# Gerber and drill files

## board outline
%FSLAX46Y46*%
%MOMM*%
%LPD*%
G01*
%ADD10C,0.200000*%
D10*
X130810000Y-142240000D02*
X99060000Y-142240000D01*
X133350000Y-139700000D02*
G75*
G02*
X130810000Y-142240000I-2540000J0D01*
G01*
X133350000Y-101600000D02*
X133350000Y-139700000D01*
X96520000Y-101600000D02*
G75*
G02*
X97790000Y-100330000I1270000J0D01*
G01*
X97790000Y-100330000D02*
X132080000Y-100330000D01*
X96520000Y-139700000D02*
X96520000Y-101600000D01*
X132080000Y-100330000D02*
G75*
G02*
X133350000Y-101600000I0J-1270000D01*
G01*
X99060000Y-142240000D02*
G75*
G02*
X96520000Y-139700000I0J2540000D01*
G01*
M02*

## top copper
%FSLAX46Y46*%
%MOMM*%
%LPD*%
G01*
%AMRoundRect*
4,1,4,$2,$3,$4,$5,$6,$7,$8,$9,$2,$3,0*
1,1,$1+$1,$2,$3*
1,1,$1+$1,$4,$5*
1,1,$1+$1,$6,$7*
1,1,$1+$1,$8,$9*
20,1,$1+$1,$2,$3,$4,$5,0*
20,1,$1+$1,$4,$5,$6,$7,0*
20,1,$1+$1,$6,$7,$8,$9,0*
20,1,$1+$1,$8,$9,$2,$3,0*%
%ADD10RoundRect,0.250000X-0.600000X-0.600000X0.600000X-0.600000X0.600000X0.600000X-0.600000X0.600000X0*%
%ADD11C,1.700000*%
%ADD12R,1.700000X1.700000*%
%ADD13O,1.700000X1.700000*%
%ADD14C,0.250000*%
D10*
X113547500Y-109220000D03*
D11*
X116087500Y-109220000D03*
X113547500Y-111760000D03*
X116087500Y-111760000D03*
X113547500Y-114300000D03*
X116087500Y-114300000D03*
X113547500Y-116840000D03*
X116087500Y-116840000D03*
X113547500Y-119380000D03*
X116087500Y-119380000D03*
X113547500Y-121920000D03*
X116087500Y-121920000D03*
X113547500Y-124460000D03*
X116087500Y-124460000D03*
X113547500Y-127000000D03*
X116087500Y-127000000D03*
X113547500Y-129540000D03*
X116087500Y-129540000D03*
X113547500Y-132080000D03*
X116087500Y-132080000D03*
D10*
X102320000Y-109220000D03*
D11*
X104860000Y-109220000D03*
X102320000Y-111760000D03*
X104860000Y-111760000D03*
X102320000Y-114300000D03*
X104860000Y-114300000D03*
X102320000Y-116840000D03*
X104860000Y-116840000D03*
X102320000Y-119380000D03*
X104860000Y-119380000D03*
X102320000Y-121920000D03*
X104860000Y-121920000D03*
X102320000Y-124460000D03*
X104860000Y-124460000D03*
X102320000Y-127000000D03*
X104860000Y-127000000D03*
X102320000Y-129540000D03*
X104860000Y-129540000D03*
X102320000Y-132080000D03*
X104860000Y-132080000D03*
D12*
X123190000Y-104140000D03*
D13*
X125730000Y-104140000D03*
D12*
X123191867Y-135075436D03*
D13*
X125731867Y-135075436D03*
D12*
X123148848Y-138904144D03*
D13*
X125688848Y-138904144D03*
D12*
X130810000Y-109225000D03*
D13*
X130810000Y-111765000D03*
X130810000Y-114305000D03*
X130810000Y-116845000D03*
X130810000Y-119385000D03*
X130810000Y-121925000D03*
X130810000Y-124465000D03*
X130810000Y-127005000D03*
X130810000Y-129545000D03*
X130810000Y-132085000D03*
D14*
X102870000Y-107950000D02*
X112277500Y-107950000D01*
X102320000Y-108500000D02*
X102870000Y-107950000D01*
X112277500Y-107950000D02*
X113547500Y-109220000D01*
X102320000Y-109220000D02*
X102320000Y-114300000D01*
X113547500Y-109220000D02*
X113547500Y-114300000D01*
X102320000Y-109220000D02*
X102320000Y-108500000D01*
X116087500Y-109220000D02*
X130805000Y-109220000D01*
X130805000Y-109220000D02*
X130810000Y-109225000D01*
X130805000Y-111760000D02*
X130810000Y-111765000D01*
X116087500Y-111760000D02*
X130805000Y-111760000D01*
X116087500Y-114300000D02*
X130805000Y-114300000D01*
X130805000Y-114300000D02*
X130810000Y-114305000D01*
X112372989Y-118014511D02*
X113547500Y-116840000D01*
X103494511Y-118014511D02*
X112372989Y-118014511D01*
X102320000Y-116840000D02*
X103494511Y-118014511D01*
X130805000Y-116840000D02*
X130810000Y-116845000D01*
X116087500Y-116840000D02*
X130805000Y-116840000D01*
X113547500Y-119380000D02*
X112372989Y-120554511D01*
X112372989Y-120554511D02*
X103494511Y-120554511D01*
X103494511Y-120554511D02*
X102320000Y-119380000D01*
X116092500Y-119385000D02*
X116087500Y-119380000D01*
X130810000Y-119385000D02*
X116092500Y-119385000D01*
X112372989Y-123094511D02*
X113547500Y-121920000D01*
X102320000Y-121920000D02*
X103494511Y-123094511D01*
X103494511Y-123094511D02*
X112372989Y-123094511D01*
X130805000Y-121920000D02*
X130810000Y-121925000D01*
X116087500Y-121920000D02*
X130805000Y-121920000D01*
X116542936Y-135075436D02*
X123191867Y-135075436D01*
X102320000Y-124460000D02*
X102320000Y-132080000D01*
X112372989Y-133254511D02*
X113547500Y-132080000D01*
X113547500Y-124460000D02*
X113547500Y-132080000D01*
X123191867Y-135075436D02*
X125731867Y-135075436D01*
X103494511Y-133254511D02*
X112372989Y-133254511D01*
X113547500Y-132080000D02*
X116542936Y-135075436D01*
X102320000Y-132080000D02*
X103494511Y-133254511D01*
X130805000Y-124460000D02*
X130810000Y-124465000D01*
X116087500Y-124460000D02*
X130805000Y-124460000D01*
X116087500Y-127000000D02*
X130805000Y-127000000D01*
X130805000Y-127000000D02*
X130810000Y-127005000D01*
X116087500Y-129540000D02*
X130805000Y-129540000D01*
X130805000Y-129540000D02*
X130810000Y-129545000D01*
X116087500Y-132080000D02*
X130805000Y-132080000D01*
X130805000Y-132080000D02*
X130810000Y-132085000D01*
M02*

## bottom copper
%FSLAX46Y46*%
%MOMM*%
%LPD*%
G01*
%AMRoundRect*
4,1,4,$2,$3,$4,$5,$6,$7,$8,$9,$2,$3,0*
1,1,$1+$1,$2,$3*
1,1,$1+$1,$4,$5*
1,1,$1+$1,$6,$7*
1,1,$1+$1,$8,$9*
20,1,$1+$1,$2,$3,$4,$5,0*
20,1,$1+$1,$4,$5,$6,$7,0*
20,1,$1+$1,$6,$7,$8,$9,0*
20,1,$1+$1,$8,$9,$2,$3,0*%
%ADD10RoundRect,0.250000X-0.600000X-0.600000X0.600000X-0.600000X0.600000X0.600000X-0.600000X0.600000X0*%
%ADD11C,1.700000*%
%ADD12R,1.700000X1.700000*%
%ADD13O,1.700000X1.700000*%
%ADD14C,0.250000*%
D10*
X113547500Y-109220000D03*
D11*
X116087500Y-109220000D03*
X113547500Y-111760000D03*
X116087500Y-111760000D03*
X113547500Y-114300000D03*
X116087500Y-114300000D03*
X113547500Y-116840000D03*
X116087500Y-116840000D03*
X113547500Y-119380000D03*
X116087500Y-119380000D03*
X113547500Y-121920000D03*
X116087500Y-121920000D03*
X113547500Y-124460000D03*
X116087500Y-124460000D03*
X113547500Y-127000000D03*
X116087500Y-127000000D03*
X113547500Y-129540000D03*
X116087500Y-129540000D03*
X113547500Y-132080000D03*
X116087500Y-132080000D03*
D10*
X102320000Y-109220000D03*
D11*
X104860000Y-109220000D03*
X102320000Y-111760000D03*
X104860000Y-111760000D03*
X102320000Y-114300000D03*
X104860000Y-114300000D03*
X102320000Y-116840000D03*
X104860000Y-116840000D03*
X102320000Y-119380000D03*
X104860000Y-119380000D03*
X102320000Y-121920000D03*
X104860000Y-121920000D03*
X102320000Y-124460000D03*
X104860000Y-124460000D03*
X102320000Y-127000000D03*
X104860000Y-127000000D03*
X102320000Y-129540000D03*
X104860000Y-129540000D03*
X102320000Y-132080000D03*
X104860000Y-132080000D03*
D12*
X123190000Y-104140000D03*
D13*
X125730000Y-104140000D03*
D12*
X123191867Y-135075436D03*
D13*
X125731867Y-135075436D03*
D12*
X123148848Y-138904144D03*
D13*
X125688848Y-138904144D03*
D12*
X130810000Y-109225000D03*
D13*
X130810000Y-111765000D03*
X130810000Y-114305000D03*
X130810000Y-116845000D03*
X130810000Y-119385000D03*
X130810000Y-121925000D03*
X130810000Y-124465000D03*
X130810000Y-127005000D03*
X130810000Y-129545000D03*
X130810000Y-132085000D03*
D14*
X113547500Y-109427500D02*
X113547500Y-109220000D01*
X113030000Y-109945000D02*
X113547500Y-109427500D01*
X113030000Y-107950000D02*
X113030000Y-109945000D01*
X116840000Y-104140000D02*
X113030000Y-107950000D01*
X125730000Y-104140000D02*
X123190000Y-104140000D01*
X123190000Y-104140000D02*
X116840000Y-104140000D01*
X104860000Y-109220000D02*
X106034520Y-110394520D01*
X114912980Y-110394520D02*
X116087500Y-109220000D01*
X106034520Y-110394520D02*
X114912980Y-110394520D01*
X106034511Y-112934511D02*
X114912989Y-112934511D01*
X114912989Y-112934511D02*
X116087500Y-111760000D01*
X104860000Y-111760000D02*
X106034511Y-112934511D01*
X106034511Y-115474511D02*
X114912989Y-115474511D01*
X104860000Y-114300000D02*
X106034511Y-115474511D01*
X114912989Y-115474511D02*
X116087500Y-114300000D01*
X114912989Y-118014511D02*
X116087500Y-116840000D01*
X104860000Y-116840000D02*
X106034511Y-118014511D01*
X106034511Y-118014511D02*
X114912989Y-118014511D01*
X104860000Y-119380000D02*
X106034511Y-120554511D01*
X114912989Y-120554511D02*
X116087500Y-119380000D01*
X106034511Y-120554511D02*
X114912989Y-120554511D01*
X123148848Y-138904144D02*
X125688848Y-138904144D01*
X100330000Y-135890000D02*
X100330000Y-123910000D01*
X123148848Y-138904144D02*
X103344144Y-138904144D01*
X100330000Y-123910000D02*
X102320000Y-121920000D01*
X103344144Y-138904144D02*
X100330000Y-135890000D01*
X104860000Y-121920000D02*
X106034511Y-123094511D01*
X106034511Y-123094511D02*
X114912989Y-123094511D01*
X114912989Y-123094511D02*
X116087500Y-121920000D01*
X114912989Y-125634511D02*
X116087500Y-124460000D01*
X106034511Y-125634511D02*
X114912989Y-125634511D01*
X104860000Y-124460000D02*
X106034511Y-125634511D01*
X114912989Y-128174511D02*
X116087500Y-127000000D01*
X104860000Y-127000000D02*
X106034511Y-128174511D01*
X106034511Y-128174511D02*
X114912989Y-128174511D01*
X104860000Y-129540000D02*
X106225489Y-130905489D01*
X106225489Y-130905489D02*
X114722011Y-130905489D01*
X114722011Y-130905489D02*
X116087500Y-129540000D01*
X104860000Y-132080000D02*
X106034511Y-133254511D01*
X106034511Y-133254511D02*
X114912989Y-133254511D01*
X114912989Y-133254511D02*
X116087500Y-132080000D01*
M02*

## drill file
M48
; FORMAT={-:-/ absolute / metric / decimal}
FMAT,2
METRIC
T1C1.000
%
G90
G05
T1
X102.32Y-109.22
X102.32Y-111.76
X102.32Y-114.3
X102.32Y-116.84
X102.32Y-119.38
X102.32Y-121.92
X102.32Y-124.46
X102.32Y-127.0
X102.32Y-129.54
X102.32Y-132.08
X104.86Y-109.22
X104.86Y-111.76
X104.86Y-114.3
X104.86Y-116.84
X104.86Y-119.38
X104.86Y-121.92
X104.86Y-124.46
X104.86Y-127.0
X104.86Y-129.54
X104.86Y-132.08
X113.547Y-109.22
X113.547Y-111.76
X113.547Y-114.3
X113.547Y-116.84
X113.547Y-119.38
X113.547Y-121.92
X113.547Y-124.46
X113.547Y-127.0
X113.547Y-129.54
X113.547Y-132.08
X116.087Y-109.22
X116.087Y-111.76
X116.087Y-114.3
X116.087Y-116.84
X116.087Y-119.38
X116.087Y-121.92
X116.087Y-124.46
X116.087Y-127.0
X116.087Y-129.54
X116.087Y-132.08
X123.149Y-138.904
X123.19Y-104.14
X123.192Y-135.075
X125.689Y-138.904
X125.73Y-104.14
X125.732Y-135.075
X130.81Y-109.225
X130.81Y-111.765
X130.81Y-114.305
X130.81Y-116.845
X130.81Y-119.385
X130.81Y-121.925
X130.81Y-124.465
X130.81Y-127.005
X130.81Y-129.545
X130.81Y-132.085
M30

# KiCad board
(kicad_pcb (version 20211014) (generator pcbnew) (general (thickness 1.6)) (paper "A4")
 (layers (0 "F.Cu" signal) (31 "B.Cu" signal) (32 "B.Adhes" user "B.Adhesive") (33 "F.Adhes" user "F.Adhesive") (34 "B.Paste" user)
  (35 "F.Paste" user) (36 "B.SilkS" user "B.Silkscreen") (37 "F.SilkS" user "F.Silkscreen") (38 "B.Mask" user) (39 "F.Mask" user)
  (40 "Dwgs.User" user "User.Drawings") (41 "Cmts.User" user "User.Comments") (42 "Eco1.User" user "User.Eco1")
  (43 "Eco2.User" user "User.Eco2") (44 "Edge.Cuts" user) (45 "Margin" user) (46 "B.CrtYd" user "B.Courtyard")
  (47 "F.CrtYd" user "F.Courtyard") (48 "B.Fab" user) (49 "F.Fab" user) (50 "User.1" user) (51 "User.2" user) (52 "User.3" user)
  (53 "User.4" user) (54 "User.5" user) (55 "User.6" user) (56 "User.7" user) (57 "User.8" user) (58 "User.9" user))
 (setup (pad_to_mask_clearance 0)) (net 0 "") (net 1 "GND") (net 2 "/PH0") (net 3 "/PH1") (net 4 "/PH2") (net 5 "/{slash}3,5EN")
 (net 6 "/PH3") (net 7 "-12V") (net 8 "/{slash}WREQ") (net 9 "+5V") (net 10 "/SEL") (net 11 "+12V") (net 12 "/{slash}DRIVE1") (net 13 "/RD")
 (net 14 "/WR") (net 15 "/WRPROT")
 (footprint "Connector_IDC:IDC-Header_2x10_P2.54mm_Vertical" (layer "F.Cu") (at 113.5475 109.22)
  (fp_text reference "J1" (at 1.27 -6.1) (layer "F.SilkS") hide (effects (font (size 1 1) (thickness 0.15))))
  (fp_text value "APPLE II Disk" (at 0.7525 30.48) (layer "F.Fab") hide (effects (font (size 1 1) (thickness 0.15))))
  (pad "1" thru_hole roundrect (at 0 0) (size 1.7 1.7) (drill 1) (layers *.Cu *.Mask) (roundrect_rratio 0.1470588235) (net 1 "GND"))
  (pad "2" thru_hole circle (at 2.54 0) (size 1.7 1.7) (drill 1) (layers *.Cu *.Mask) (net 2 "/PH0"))
  (pad "3" thru_hole circle (at 0 2.54) (size 1.7 1.7) (drill 1) (layers *.Cu *.Mask) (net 1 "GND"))
  (pad "4" thru_hole circle (at 2.54 2.54) (size 1.7 1.7) (drill 1) (layers *.Cu *.Mask) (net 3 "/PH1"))
  (pad "5" thru_hole circle (at 0 5.08) (size 1.7 1.7) (drill 1) (layers *.Cu *.Mask) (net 1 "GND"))
  (pad "6" thru_hole circle (at 2.54 5.08) (size 1.7 1.7) (drill 1) (layers *.Cu *.Mask) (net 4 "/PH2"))
  (pad "7" thru_hole circle (at 0 7.62) (size 1.7 1.7) (drill 1) (layers *.Cu *.Mask) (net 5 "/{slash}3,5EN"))
  (pad "8" thru_hole circle (at 2.54 7.62) (size 1.7 1.7) (drill 1) (layers *.Cu *.Mask) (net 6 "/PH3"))
  (pad "9" thru_hole circle (at 0 10.16) (size 1.7 1.7) (drill 1) (layers *.Cu *.Mask) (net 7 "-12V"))
  (pad "10" thru_hole circle (at 2.54 10.16) (size 1.7 1.7) (drill 1) (layers *.Cu *.Mask) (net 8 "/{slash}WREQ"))
  (pad "11" thru_hole circle (at 0 12.7) (size 1.7 1.7) (drill 1) (layers *.Cu *.Mask) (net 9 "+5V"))
  (pad "12" thru_hole circle (at 2.54 12.7) (size 1.7 1.7) (drill 1) (layers *.Cu *.Mask) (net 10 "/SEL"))
  (pad "13" thru_hole circle (at 0 15.24) (size 1.7 1.7) (drill 1) (layers *.Cu *.Mask) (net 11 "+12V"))
  (pad "14" thru_hole circle (at 2.54 15.24) (size 1.7 1.7) (drill 1) (layers *.Cu *.Mask) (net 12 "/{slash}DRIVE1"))
  (pad "15" thru_hole circle (at 0 17.78) (size 1.7 1.7) (drill 1) (layers *.Cu *.Mask) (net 11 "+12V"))
  (pad "16" thru_hole circle (at 2.54 17.78) (size 1.7 1.7) (drill 1) (layers *.Cu *.Mask) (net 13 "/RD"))
  (pad "17" thru_hole circle (at 0 20.32) (size 1.7 1.7) (drill 1) (layers *.Cu *.Mask) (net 11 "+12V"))
  (pad "18" thru_hole circle (at 2.54 20.32) (size 1.7 1.7) (drill 1) (layers *.Cu *.Mask) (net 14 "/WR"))
  (pad "19" thru_hole circle (at 0 22.86) (size 1.7 1.7) (drill 1) (layers *.Cu *.Mask) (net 11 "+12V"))
  (pad "20" thru_hole circle (at 2.54 22.86) (size 1.7 1.7) (drill 1) (layers *.Cu *.Mask) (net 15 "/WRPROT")))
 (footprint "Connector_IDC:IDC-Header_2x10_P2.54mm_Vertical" (layer "F.Cu") (at 102.32 109.22)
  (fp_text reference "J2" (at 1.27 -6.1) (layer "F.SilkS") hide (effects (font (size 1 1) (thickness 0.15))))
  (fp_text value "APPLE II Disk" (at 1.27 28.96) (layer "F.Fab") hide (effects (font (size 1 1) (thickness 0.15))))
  (pad "1" thru_hole roundrect (at 0 0) (size 1.7 1.7) (drill 1) (layers *.Cu *.Mask) (roundrect_rratio 0.1470588235) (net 1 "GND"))
  (pad "2" thru_hole circle (at 2.54 0) (size 1.7 1.7) (drill 1) (layers *.Cu *.Mask) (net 2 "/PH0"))
  (pad "3" thru_hole circle (at 0 2.54) (size 1.7 1.7) (drill 1) (layers *.Cu *.Mask) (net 1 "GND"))
  (pad "4" thru_hole circle (at 2.54 2.54) (size 1.7 1.7) (drill 1) (layers *.Cu *.Mask) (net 3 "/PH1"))
  (pad "5" thru_hole circle (at 0 5.08) (size 1.7 1.7) (drill 1) (layers *.Cu *.Mask) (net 1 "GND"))
  (pad "6" thru_hole circle (at 2.54 5.08) (size 1.7 1.7) (drill 1) (layers *.Cu *.Mask) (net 4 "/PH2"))
  (pad "7" thru_hole circle (at 0 7.62) (size 1.7 1.7) (drill 1) (layers *.Cu *.Mask) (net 5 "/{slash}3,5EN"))
  (pad "8" thru_hole circle (at 2.54 7.62) (size 1.7 1.7) (drill 1) (layers *.Cu *.Mask) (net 6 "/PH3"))
  (pad "9" thru_hole circle (at 0 10.16) (size 1.7 1.7) (drill 1) (layers *.Cu *.Mask) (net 7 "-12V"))
  (pad "10" thru_hole circle (at 2.54 10.16) (size 1.7 1.7) (drill 1) (layers *.Cu *.Mask) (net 8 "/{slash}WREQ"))
  (pad "11" thru_hole circle (at 0 12.7) (size 1.7 1.7) (drill 1) (layers *.Cu *.Mask) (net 9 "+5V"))
  (pad "12" thru_hole circle (at 2.54 12.7) (size 1.7 1.7) (drill 1) (layers *.Cu *.Mask) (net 10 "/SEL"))
  (pad "13" thru_hole circle (at 0 15.24) (size 1.7 1.7) (drill 1) (layers *.Cu *.Mask) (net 11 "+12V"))
  (pad "14" thru_hole circle (at 2.54 15.24) (size 1.7 1.7) (drill 1) (layers *.Cu *.Mask) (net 12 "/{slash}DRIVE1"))
  (pad "15" thru_hole circle (at 0 17.78) (size 1.7 1.7) (drill 1) (layers *.Cu *.Mask) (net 11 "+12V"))
  (pad "16" thru_hole circle (at 2.54 17.78) (size 1.7 1.7) (drill 1) (layers *.Cu *.Mask) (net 13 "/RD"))
  (pad "17" thru_hole circle (at 0 20.32) (size 1.7 1.7) (drill 1) (layers *.Cu *.Mask) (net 11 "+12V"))
  (pad "18" thru_hole circle (at 2.54 20.32) (size 1.7 1.7) (drill 1) (layers *.Cu *.Mask) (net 14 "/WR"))
  (pad "19" thru_hole circle (at 0 22.86) (size 1.7 1.7) (drill 1) (layers *.Cu *.Mask) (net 11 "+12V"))
  (pad "20" thru_hole circle (at 2.54 22.86) (size 1.7 1.7) (drill 1) (layers *.Cu *.Mask) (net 15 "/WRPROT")))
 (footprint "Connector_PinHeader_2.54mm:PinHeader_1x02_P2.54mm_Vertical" (layer "F.Cu") (at 123.19 104.14 90)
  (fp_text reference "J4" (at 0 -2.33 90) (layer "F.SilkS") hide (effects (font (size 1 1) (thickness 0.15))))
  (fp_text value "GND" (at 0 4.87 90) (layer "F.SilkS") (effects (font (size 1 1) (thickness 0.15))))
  (pad "1" thru_hole rect (at 0 0 90) (size 1.7 1.7) (drill 1) (layers *.Cu *.Mask) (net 1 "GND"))
  (pad "2" thru_hole oval (at 0 2.54 90) (size 1.7 1.7) (drill 1) (layers *.Cu *.Mask) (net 1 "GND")))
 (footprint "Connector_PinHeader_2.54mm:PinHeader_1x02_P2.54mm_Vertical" (layer "F.Cu") (at 123.191867 135.075436 90)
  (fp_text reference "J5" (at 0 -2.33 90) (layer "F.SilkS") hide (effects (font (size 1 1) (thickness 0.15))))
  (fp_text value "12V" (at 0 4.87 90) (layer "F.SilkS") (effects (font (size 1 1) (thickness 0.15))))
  (pad "1" thru_hole rect (at 0 0 90) (size 1.7 1.7) (drill 1) (layers *.Cu *.Mask) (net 11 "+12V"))
  (pad "2" thru_hole oval (at 0 2.54 90) (size 1.7 1.7) (drill 1) (layers *.Cu *.Mask) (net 11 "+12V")))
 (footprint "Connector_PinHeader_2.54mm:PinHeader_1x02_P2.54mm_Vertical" (layer "F.Cu") (at 123.148848 138.904144 90)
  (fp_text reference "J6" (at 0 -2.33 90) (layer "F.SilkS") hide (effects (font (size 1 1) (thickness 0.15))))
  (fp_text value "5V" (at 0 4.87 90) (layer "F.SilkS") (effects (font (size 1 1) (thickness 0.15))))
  (pad "1" thru_hole rect (at 0 0 90) (size 1.7 1.7) (drill 1) (layers *.Cu *.Mask) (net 9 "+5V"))
  (pad "2" thru_hole oval (at 0 2.54 90) (size 1.7 1.7) (drill 1) (layers *.Cu *.Mask) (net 9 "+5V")))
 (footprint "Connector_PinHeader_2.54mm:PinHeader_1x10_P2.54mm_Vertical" (layer "F.Cu") (at 130.81 109.225)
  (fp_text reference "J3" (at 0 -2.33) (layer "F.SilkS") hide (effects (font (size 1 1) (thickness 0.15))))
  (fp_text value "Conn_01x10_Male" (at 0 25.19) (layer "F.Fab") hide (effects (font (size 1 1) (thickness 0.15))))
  (pad "1" thru_hole rect (at 0 0) (size 1.7 1.7) (drill 1) (layers *.Cu *.Mask) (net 2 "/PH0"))
  (pad "2" thru_hole oval (at 0 2.54) (size 1.7 1.7) (drill 1) (layers *.Cu *.Mask) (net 3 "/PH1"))
  (pad "3" thru_hole oval (at 0 5.08) (size 1.7 1.7) (drill 1) (layers *.Cu *.Mask) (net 4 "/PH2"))
  (pad "4" thru_hole oval (at 0 7.62) (size 1.7 1.7) (drill 1) (layers *.Cu *.Mask) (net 6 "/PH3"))
  (pad "5" thru_hole oval (at 0 10.16) (size 1.7 1.7) (drill 1) (layers *.Cu *.Mask) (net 8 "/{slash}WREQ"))
  (pad "6" thru_hole oval (at 0 12.7) (size 1.7 1.7) (drill 1) (layers *.Cu *.Mask) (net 10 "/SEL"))
  (pad "7" thru_hole oval (at 0 15.24) (size 1.7 1.7) (drill 1) (layers *.Cu *.Mask) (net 12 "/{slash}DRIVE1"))
  (pad "8" thru_hole oval (at 0 17.78) (size 1.7 1.7) (drill 1) (layers *.Cu *.Mask) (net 13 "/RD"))
  (pad "9" thru_hole oval (at 0 20.32) (size 1.7 1.7) (drill 1) (layers *.Cu *.Mask) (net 14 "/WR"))
  (pad "10" thru_hole oval (at 0 22.86) (size 1.7 1.7) (drill 1) (layers *.Cu *.Mask) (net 15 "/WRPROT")))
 (gr_line (start 130.81 142.24) (end 99.06 142.24) (layer "Edge.Cuts") (width 0.2))
 (gr_arc (start 133.35 139.7) (mid 132.606051 141.496051) (end 130.81 142.24) (layer "Edge.Cuts") (width 0.2))
 (gr_line (start 133.35 101.6) (end 133.35 139.7) (layer "Edge.Cuts") (width 0.2))
 (gr_arc (start 96.52 101.6) (mid 96.891974 100.701974) (end 97.79 100.33) (layer "Edge.Cuts") (width 0.2))
 (gr_line (start 97.79 100.33) (end 132.08 100.33) (layer "Edge.Cuts") (width 0.2))
 (gr_line (start 96.52 139.7) (end 96.52 101.6) (layer "Edge.Cuts") (width 0.2))
 (gr_arc (start 132.08 100.33) (mid 132.978026 100.701974) (end 133.35 101.6) (layer "Edge.Cuts") (width 0.2))
 (gr_arc (start 99.06 142.24) (mid 97.263949 141.496051) (end 96.52 139.7) (layer "Edge.Cuts") (width 0.2))
 (segment (start 102.87 107.95) (end 112.2775 107.95) (width 0.25) (layer "F.Cu") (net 1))
 (segment (start 102.32 108.5) (end 102.87 107.95) (width 0.25) (layer "F.Cu") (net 1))
 (segment (start 112.2775 107.95) (end 113.5475 109.22) (width 0.25) (layer "F.Cu") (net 1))
 (segment (start 102.32 109.22) (end 102.32 114.3) (width 0.25) (layer "F.Cu") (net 1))
 (segment (start 113.5475 109.22) (end 113.5475 114.3) (width 0.25) (layer "F.Cu") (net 1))
 (segment (start 102.32 109.22) (end 102.32 108.5) (width 0.25) (layer "F.Cu") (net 1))
 (segment (start 113.5475 109.4275) (end 113.5475 109.22) (width 0.25) (layer "B.Cu") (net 1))
 (segment (start 113.03 109.945) (end 113.5475 109.4275) (width 0.25) (layer "B.Cu") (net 1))
 (segment (start 113.03 107.95) (end 113.03 109.945) (width 0.25) (layer "B.Cu") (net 1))
 (segment (start 116.84 104.14) (end 113.03 107.95) (width 0.25) (layer "B.Cu") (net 1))
 (segment (start 125.73 104.14) (end 123.19 104.14) (width 0.25) (layer "B.Cu") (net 1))
 (segment (start 123.19 104.14) (end 116.84 104.14) (width 0.25) (layer "B.Cu") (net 1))
 (segment (start 116.0875 109.22) (end 130.805 109.22) (width 0.25) (layer "F.Cu") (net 2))
 (segment (start 130.805 109.22) (end 130.81 109.225) (width 0.25) (layer "F.Cu") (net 2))
 (segment (start 104.86 109.22) (end 106.03452 110.39452) (width 0.25) (layer "B.Cu") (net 2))
 (segment (start 114.91298 110.39452) (end 116.0875 109.22) (width 0.25) (layer "B.Cu") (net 2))
 (segment (start 106.03452 110.39452) (end 114.91298 110.39452) (width 0.25) (layer "B.Cu") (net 2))
 (segment (start 130.805 111.76) (end 130.81 111.765) (width 0.25) (layer "F.Cu") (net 3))
 (segment (start 116.0875 111.76) (end 130.805 111.76) (width 0.25) (layer "F.Cu") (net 3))
 (segment (start 106.034511 112.934511) (end 114.912989 112.934511) (width 0.25) (layer "B.Cu") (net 3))
 (segment (start 114.912989 112.934511) (end 116.0875 111.76) (width 0.25) (layer "B.Cu") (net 3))
 (segment (start 104.86 111.76) (end 106.034511 112.934511) (width 0.25) (layer "B.Cu") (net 3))
 (segment (start 116.0875 114.3) (end 130.805 114.3) (width 0.25) (layer "F.Cu") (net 4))
 (segment (start 130.805 114.3) (end 130.81 114.305) (width 0.25) (layer "F.Cu") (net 4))
 (segment (start 106.034511 115.474511) (end 114.912989 115.474511) (width 0.25) (layer "B.Cu") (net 4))
 (segment (start 104.86 114.3) (end 106.034511 115.474511) (width 0.25) (layer "B.Cu") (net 4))
 (segment (start 114.912989 115.474511) (end 116.0875 114.3) (width 0.25) (layer "B.Cu") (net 4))
 (segment (start 112.372989 118.014511) (end 113.5475 116.84) (width 0.25) (layer "F.Cu") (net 5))
 (segment (start 103.494511 118.014511) (end 112.372989 118.014511) (width 0.25) (layer "F.Cu") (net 5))
 (segment (start 102.32 116.84) (end 103.494511 118.014511) (width 0.25) (layer "F.Cu") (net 5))
 (segment (start 130.805 116.84) (end 130.81 116.845) (width 0.25) (layer "F.Cu") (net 6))
 (segment (start 116.0875 116.84) (end 130.805 116.84) (width 0.25) (layer "F.Cu") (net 6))
 (segment (start 114.912989 118.014511) (end 116.0875 116.84) (width 0.25) (layer "B.Cu") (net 6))
 (segment (start 104.86 116.84) (end 106.034511 118.014511) (width 0.25) (layer "B.Cu") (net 6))
 (segment (start 106.034511 118.014511) (end 114.912989 118.014511) (width 0.25) (layer "B.Cu") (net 6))
 (segment (start 113.5475 119.38) (end 112.372989 120.554511) (width 0.25) (layer "F.Cu") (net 7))
 (segment (start 112.372989 120.554511) (end 103.494511 120.554511) (width 0.25) (layer "F.Cu") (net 7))
 (segment (start 103.494511 120.554511) (end 102.32 119.38) (width 0.25) (layer "F.Cu") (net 7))
 (segment (start 116.0925 119.385) (end 116.0875 119.38) (width 0.25) (layer "F.Cu") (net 8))
 (segment (start 130.81 119.385) (end 116.0925 119.385) (width 0.25) (layer "F.Cu") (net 8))
 (segment (start 104.86 119.38) (end 106.034511 120.554511) (width 0.25) (layer "B.Cu") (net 8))
 (segment (start 114.912989 120.554511) (end 116.0875 119.38) (width 0.25) (layer "B.Cu") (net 8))
 (segment (start 106.034511 120.554511) (end 114.912989 120.554511) (width 0.25) (layer "B.Cu") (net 8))
 (segment (start 112.372989 123.094511) (end 113.5475 121.92) (width 0.25) (layer "F.Cu") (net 9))
 (segment (start 102.32 121.92) (end 103.494511 123.094511) (width 0.25) (layer "F.Cu") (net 9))
 (segment (start 103.494511 123.094511) (end 112.372989 123.094511) (width 0.25) (layer "F.Cu") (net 9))
 (segment (start 123.148848 138.904144) (end 125.688848 138.904144) (width 0.25) (layer "B.Cu") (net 9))
 (segment (start 100.33 135.89) (end 100.33 123.91) (width 0.25) (layer "B.Cu") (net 9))
 (segment (start 123.148848 138.904144) (end 103.344144 138.904144) (width 0.25) (layer "B.Cu") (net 9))
 (segment (start 100.33 123.91) (end 102.32 121.92) (width 0.25) (layer "B.Cu") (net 9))
 (segment (start 103.344144 138.904144) (end 100.33 135.89) (width 0.25) (layer "B.Cu") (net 9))
 (segment (start 130.805 121.92) (end 130.81 121.925) (width 0.25) (layer "F.Cu") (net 10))
 (segment (start 116.0875 121.92) (end 130.805 121.92) (width 0.25) (layer "F.Cu") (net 10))
 (segment (start 104.86 121.92) (end 106.034511 123.094511) (width 0.25) (layer "B.Cu") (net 10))
 (segment (start 106.034511 123.094511) (end 114.912989 123.094511) (width 0.25) (layer "B.Cu") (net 10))
 (segment (start 114.912989 123.094511) (end 116.0875 121.92) (width 0.25) (layer "B.Cu") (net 10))
 (segment (start 116.542936 135.075436) (end 123.191867 135.075436) (width 0.25) (layer "F.Cu") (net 11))
 (segment (start 102.32 124.46) (end 102.32 132.08) (width 0.25) (layer "F.Cu") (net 11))
 (segment (start 112.372989 133.254511) (end 113.5475 132.08) (width 0.25) (layer "F.Cu") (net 11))
 (segment (start 113.5475 124.46) (end 113.5475 132.08) (width 0.25) (layer "F.Cu") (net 11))
 (segment (start 123.191867 135.075436) (end 125.731867 135.075436) (width 0.25) (layer "F.Cu") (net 11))
 (segment (start 103.494511 133.254511) (end 112.372989 133.254511) (width 0.25) (layer "F.Cu") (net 11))
 (segment (start 113.5475 132.08) (end 116.542936 135.075436) (width 0.25) (layer "F.Cu") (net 11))
 (segment (start 102.32 132.08) (end 103.494511 133.254511) (width 0.25) (layer "F.Cu") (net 11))
 (segment (start 130.805 124.46) (end 130.81 124.465) (width 0.25) (layer "F.Cu") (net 12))
 (segment (start 116.0875 124.46) (end 130.805 124.46) (width 0.25) (layer "F.Cu") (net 12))
 (segment (start 114.912989 125.634511) (end 116.0875 124.46) (width 0.25) (layer "B.Cu") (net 12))
 (segment (start 106.034511 125.634511) (end 114.912989 125.634511) (width 0.25) (layer "B.Cu") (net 12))
 (segment (start 104.86 124.46) (end 106.034511 125.634511) (width 0.25) (layer "B.Cu") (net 12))
 (segment (start 116.0875 127) (end 130.805 127) (width 0.25) (layer "F.Cu") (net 13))
 (segment (start 130.805 127) (end 130.81 127.005) (width 0.25) (layer "F.Cu") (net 13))
 (segment (start 114.912989 128.174511) (end 116.0875 127) (width 0.25) (layer "B.Cu") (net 13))
 (segment (start 104.86 127) (end 106.034511 128.174511) (width 0.25) (layer "B.Cu") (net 13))
 (segment (start 106.034511 128.174511) (end 114.912989 128.174511) (width 0.25) (layer "B.Cu") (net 13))
 (segment (start 116.0875 129.54) (end 130.805 129.54) (width 0.25) (layer "F.Cu") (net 14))
 (segment (start 130.805 129.54) (end 130.81 129.545) (width 0.25) (layer "F.Cu") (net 14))
 (segment (start 104.86 129.54) (end 106.225489 130.905489) (width 0.25) (layer "B.Cu") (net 14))
 (segment (start 106.225489 130.905489) (end 114.722011 130.905489) (width 0.25) (layer "B.Cu") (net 14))
 (segment (start 114.722011 130.905489) (end 116.0875 129.54) (width 0.25) (layer "B.Cu") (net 14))
 (segment (start 116.0875 132.08) (end 130.805 132.08) (width 0.25) (layer "F.Cu") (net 15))
 (segment (start 130.805 132.08) (end 130.81 132.085) (width 0.25) (layer "F.Cu") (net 15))
 (segment (start 104.86 132.08) (end 106.034511 133.254511) (width 0.25) (layer "B.Cu") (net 15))
 (segment (start 106.034511 133.254511) (end 114.912989 133.254511) (width 0.25) (layer "B.Cu") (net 15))
 (segment (start 114.912989 133.254511) (end 116.0875 132.08) (width 0.25) (layer "B.Cu") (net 15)))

